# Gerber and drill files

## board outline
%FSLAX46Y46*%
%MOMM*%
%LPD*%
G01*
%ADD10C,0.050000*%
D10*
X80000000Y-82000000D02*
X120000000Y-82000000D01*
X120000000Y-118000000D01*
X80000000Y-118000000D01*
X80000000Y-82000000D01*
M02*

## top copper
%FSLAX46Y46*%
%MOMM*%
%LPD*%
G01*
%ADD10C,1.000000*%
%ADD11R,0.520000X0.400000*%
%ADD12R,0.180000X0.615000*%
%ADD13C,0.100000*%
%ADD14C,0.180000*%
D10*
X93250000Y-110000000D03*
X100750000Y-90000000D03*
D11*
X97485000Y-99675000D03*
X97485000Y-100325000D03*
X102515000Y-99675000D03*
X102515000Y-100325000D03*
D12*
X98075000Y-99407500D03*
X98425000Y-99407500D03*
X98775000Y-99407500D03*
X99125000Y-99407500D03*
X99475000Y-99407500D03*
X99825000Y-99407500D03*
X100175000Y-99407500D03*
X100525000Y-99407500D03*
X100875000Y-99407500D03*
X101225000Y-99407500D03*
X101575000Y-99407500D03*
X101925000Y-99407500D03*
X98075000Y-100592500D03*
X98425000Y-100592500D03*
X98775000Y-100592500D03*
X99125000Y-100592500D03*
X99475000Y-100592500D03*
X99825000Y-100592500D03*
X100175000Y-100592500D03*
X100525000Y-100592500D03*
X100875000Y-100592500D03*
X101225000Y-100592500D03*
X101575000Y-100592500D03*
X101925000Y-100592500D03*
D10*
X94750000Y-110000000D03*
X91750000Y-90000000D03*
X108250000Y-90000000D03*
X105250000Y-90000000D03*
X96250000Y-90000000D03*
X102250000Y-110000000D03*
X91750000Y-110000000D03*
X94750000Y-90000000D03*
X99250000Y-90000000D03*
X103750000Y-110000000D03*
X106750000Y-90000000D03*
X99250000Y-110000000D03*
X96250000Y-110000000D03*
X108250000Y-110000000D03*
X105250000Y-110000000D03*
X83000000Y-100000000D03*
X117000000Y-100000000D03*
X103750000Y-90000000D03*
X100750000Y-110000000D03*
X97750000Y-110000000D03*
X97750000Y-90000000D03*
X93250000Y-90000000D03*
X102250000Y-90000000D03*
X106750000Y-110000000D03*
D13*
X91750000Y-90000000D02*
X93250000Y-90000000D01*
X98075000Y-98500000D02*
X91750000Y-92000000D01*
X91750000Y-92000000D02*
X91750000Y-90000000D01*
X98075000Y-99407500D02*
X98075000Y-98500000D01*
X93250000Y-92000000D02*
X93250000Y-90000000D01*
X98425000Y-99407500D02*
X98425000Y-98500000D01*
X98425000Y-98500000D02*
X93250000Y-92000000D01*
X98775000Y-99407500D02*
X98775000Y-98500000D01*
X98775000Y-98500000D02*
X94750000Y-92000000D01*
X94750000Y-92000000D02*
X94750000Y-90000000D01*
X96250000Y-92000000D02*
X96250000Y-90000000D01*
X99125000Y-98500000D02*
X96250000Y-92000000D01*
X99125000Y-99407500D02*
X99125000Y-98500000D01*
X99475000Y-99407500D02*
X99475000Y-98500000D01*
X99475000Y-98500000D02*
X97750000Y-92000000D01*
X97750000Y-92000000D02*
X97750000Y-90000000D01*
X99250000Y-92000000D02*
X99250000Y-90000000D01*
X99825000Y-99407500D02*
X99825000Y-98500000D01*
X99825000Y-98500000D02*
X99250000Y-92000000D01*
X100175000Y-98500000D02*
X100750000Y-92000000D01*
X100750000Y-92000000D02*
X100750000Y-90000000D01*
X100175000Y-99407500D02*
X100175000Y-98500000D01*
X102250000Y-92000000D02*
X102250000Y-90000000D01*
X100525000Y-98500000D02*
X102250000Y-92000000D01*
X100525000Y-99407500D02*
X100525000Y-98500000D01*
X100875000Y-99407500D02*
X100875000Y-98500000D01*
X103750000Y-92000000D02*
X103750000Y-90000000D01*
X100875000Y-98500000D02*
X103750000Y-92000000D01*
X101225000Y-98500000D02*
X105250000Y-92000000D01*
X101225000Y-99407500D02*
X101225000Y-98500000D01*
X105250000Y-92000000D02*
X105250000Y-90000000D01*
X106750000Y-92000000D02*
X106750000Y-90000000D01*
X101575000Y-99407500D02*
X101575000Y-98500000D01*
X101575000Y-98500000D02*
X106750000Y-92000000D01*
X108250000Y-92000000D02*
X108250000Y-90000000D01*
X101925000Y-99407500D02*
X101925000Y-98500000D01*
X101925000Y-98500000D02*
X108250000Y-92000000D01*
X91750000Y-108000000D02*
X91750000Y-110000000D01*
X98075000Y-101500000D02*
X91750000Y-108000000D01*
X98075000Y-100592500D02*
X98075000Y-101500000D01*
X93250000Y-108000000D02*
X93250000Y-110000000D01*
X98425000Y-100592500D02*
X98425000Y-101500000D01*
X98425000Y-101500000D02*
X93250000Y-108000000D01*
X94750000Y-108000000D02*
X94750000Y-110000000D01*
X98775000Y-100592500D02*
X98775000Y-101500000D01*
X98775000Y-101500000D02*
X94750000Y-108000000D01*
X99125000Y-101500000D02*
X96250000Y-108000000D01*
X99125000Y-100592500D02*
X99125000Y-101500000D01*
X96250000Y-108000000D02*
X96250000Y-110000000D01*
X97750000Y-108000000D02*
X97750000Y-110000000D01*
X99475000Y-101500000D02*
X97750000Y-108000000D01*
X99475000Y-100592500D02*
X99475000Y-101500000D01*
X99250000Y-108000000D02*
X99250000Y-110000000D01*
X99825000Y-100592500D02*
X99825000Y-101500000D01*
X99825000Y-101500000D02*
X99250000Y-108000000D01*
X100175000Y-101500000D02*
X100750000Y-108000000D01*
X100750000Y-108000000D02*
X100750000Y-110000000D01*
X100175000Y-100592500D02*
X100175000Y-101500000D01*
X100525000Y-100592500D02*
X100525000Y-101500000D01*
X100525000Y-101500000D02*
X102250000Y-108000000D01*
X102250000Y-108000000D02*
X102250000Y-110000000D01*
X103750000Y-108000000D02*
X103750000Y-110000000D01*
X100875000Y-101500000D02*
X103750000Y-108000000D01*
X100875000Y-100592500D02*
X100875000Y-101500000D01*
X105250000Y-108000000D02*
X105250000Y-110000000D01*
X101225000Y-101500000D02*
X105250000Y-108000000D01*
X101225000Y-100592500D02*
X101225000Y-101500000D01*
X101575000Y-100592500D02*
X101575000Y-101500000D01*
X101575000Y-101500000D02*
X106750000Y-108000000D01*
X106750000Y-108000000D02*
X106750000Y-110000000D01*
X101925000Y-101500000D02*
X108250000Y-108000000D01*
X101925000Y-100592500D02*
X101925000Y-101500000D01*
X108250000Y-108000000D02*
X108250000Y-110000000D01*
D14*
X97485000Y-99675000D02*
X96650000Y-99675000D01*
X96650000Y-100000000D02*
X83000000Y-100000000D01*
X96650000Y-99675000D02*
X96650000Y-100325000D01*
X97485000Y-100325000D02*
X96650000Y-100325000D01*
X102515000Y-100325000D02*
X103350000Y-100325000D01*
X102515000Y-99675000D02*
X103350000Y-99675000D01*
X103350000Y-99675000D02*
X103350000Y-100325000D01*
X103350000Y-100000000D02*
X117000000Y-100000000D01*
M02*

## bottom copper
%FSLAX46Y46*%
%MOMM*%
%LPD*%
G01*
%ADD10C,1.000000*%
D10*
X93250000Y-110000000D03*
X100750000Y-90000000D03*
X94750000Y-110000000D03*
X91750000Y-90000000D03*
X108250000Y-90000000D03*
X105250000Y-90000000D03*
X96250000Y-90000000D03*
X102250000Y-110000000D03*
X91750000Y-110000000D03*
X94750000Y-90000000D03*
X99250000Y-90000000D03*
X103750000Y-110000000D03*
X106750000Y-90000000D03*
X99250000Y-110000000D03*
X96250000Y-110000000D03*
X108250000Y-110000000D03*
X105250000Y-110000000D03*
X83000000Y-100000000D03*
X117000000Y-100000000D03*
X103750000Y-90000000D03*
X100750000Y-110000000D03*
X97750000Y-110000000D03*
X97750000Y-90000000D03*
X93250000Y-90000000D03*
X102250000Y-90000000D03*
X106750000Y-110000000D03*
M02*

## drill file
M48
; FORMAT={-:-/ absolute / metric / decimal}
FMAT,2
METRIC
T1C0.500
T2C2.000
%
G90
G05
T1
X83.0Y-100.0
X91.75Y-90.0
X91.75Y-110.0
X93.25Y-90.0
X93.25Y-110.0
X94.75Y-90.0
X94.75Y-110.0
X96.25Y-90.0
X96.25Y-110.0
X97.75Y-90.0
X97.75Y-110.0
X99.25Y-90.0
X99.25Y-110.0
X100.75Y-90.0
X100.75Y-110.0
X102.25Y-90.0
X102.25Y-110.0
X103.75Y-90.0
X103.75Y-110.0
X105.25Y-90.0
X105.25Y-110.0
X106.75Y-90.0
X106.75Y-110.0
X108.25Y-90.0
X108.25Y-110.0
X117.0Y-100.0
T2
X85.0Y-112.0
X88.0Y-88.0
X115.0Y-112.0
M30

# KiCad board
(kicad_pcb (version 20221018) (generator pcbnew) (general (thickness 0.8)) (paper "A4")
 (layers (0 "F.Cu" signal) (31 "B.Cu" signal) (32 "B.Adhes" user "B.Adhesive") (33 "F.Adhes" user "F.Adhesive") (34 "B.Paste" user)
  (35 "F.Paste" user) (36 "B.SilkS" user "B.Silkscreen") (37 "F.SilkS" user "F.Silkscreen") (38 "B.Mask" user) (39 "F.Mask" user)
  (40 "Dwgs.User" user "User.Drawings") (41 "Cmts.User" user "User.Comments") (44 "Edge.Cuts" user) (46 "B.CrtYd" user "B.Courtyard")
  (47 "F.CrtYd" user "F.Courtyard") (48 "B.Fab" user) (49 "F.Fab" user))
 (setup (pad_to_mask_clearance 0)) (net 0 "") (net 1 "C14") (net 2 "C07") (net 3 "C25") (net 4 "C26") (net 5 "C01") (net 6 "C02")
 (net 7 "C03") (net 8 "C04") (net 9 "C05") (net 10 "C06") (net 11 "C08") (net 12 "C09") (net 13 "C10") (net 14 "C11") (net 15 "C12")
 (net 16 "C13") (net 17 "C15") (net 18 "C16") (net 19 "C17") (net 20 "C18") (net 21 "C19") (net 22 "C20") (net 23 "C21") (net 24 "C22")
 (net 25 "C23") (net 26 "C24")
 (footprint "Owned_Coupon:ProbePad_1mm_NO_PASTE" (layer "F.Cu") (at 93.25 110)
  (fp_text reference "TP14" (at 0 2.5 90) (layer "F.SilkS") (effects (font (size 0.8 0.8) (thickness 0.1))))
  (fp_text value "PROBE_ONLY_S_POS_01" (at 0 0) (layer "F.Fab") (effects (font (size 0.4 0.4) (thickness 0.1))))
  (pad "1" thru_hole circle (at 0 0) (size 1 1) (drill 0.5) (layers "*.Cu" "*.Mask") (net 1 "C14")))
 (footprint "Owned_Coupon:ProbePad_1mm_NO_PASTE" (layer "F.Cu") (at 100.75 90)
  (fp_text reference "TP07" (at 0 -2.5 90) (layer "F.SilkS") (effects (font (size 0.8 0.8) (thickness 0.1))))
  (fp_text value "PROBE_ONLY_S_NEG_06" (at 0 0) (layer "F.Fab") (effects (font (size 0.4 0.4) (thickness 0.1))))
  (pad "1" thru_hole circle (at 0 0) (size 1 1) (drill 0.5) (layers "*.Cu" "*.Mask") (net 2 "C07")))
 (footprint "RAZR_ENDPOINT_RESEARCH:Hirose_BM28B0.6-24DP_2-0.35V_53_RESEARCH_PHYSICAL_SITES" (layer "F.Cu") (at 100 100)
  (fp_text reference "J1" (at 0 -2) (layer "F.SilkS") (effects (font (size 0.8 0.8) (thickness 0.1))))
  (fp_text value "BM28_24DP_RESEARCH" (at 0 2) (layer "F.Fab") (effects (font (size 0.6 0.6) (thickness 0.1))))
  (pad "P_L" smd rect (at -2.515 -0.325) (size 0.52 0.4) (layers "F.Cu" "F.Mask") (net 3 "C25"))
  (pad "P_L" smd rect (at -2.515 0.325) (size 0.52 0.4) (layers "F.Cu" "F.Mask") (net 3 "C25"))
  (pad "P_R" smd rect (at 2.515 -0.325) (size 0.52 0.4) (layers "F.Cu" "F.Mask") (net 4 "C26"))
  (pad "P_R" smd rect (at 2.515 0.325) (size 0.52 0.4) (layers "F.Cu" "F.Mask") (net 4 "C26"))
  (pad "S_NEG_00" smd rect (at -1.925 -0.5925) (size 0.18 0.615) (layers "F.Cu" "F.Mask") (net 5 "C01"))
  (pad "S_NEG_01" smd rect (at -1.575 -0.5925) (size 0.18 0.615) (layers "F.Cu" "F.Mask") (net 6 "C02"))
  (pad "S_NEG_02" smd rect (at -1.225 -0.5925) (size 0.18 0.615) (layers "F.Cu" "F.Mask") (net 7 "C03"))
  (pad "S_NEG_03" smd rect (at -0.875 -0.5925) (size 0.18 0.615) (layers "F.Cu" "F.Mask") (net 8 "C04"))
  (pad "S_NEG_04" smd rect (at -0.525 -0.5925) (size 0.18 0.615) (layers "F.Cu" "F.Mask") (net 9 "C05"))
  (pad "S_NEG_05" smd rect (at -0.175 -0.5925) (size 0.18 0.615) (layers "F.Cu" "F.Mask") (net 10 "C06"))
  (pad "S_NEG_06" smd rect (at 0.175 -0.5925) (size 0.18 0.615) (layers "F.Cu" "F.Mask") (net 2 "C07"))
  (pad "S_NEG_07" smd rect (at 0.525 -0.5925) (size 0.18 0.615) (layers "F.Cu" "F.Mask") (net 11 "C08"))
  (pad "S_NEG_08" smd rect (at 0.875 -0.5925) (size 0.18 0.615) (layers "F.Cu" "F.Mask") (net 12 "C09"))
  (pad "S_NEG_09" smd rect (at 1.225 -0.5925) (size 0.18 0.615) (layers "F.Cu" "F.Mask") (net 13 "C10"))
  (pad "S_NEG_10" smd rect (at 1.575 -0.5925) (size 0.18 0.615) (layers "F.Cu" "F.Mask") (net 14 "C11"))
  (pad "S_NEG_11" smd rect (at 1.925 -0.5925) (size 0.18 0.615) (layers "F.Cu" "F.Mask") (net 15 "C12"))
  (pad "S_POS_00" smd rect (at -1.925 0.5925) (size 0.18 0.615) (layers "F.Cu" "F.Mask") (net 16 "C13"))
  (pad "S_POS_01" smd rect (at -1.575 0.5925) (size 0.18 0.615) (layers "F.Cu" "F.Mask") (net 1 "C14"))
  (pad "S_POS_02" smd rect (at -1.225 0.5925) (size 0.18 0.615) (layers "F.Cu" "F.Mask") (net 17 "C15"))
  (pad "S_POS_03" smd rect (at -0.875 0.5925) (size 0.18 0.615) (layers "F.Cu" "F.Mask") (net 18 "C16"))
  (pad "S_POS_04" smd rect (at -0.525 0.5925) (size 0.18 0.615) (layers "F.Cu" "F.Mask") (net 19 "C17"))
  (pad "S_POS_05" smd rect (at -0.175 0.5925) (size 0.18 0.615) (layers "F.Cu" "F.Mask") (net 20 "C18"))
  (pad "S_POS_06" smd rect (at 0.175 0.5925) (size 0.18 0.615) (layers "F.Cu" "F.Mask") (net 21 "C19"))
  (pad "S_POS_07" smd rect (at 0.525 0.5925) (size 0.18 0.615) (layers "F.Cu" "F.Mask") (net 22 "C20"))
  (pad "S_POS_08" smd rect (at 0.875 0.5925) (size 0.18 0.615) (layers "F.Cu" "F.Mask") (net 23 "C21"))
  (pad "S_POS_09" smd rect (at 1.225 0.5925) (size 0.18 0.615) (layers "F.Cu" "F.Mask") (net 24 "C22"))
  (pad "S_POS_10" smd rect (at 1.575 0.5925) (size 0.18 0.615) (layers "F.Cu" "F.Mask") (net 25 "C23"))
  (pad "S_POS_11" smd rect (at 1.925 0.5925) (size 0.18 0.615) (layers "F.Cu" "F.Mask") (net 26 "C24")))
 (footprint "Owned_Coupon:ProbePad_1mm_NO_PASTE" (layer "F.Cu") (at 94.75 110)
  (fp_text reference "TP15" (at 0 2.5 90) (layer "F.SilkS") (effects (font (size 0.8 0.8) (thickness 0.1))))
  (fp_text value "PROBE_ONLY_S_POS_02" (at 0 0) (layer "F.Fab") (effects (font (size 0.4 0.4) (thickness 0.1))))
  (pad "1" thru_hole circle (at 0 0) (size 1 1) (drill 0.5) (layers "*.Cu" "*.Mask") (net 17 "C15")))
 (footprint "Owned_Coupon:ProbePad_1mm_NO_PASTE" (layer "F.Cu") (at 91.75 90)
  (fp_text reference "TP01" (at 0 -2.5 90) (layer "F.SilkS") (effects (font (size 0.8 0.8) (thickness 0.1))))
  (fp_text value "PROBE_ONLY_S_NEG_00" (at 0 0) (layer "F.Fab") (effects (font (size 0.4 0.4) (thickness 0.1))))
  (pad "1" thru_hole circle (at 0 0) (size 1 1) (drill 0.5) (layers "*.Cu" "*.Mask") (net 5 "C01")))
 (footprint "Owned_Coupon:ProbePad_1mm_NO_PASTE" (layer "F.Cu") (at 108.25 90)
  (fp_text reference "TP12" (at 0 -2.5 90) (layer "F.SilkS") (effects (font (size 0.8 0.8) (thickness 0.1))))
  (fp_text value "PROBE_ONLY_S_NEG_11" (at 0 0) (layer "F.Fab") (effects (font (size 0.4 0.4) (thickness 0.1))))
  (pad "1" thru_hole circle (at 0 0) (size 1 1) (drill 0.5) (layers "*.Cu" "*.Mask") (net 15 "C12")))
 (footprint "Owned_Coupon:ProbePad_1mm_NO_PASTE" (layer "F.Cu") (at 105.25 90)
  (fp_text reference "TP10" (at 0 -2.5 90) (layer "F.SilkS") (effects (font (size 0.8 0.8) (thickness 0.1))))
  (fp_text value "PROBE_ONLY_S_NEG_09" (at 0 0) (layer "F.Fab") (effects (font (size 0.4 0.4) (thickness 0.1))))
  (pad "1" thru_hole circle (at 0 0) (size 1 1) (drill 0.5) (layers "*.Cu" "*.Mask") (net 13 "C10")))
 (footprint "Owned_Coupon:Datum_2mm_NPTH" (layer "F.Cu") (at 88 88)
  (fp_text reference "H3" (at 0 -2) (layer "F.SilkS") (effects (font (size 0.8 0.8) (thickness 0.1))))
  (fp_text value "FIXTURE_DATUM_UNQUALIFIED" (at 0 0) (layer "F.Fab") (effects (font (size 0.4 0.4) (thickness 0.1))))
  (pad "" np_thru_hole circle (at 0 0) (size 2 2) (drill 2) (layers "*.Cu" "*.Mask")))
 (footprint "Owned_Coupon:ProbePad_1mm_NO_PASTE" (layer "F.Cu") (at 96.25 90)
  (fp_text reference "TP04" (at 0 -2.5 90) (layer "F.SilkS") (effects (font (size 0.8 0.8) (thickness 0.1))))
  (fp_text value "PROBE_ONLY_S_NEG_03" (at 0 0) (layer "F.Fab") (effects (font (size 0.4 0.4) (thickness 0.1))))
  (pad "1" thru_hole circle (at 0 0) (size 1 1) (drill 0.5) (layers "*.Cu" "*.Mask") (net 8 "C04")))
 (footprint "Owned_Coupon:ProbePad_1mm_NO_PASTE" (layer "F.Cu") (at 102.25 110)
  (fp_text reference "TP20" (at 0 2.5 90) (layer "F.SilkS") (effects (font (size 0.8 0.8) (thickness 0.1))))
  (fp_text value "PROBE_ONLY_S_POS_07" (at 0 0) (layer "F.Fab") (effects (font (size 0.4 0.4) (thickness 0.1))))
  (pad "1" thru_hole circle (at 0 0) (size 1 1) (drill 0.5) (layers "*.Cu" "*.Mask") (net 22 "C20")))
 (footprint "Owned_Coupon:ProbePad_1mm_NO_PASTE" (layer "F.Cu") (at 91.75 110)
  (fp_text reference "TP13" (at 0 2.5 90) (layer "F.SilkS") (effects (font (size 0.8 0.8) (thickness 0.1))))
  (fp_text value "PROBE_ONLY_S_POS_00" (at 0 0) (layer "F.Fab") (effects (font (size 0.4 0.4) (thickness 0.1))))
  (pad "1" thru_hole circle (at 0 0) (size 1 1) (drill 0.5) (layers "*.Cu" "*.Mask") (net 16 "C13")))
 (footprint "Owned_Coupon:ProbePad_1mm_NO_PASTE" (layer "F.Cu") (at 94.75 90)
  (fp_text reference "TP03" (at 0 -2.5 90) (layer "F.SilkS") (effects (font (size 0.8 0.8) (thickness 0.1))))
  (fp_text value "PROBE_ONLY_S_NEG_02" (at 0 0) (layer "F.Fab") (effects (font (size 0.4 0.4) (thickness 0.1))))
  (pad "1" thru_hole circle (at 0 0) (size 1 1) (drill 0.5) (layers "*.Cu" "*.Mask") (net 7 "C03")))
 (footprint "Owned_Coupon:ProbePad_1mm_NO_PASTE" (layer "F.Cu") (at 99.25 90)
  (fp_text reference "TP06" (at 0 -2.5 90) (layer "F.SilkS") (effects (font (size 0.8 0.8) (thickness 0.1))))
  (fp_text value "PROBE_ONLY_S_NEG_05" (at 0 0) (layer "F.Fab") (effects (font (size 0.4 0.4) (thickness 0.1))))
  (pad "1" thru_hole circle (at 0 0) (size 1 1) (drill 0.5) (layers "*.Cu" "*.Mask") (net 10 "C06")))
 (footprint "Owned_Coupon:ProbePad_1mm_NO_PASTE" (layer "F.Cu") (at 103.75 110)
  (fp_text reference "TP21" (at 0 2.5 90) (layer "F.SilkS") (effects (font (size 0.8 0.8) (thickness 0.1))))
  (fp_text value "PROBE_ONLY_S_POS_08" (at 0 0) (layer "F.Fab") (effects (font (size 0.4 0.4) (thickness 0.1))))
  (pad "1" thru_hole circle (at 0 0) (size 1 1) (drill 0.5) (layers "*.Cu" "*.Mask") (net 23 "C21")))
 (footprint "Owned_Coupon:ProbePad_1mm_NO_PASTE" (layer "F.Cu") (at 106.75 90)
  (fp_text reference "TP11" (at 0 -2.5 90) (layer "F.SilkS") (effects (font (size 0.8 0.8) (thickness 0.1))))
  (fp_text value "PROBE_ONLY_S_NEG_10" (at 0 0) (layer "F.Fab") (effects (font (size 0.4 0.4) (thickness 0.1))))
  (pad "1" thru_hole circle (at 0 0) (size 1 1) (drill 0.5) (layers "*.Cu" "*.Mask") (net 14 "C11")))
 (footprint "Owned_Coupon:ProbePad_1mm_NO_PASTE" (layer "F.Cu") (at 99.25 110)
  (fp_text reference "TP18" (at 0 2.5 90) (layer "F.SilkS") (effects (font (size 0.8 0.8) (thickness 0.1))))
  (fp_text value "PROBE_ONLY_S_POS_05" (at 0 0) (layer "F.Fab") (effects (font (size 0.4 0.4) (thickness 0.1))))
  (pad "1" thru_hole circle (at 0 0) (size 1 1) (drill 0.5) (layers "*.Cu" "*.Mask") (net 20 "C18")))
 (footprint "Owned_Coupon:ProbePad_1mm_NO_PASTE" (layer "F.Cu") (at 96.25 110)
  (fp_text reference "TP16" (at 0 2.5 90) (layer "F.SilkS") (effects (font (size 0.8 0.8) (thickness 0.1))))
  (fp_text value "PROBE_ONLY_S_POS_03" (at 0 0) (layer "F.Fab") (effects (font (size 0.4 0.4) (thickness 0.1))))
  (pad "1" thru_hole circle (at 0 0) (size 1 1) (drill 0.5) (layers "*.Cu" "*.Mask") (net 18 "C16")))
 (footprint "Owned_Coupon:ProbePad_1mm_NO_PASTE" (layer "F.Cu") (at 108.25 110)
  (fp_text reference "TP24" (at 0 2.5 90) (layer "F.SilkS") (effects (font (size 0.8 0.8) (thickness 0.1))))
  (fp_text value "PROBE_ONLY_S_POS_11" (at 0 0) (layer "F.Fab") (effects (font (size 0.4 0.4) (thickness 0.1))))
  (pad "1" thru_hole circle (at 0 0) (size 1 1) (drill 0.5) (layers "*.Cu" "*.Mask") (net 26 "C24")))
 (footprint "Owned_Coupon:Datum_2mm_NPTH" (layer "F.Cu") (at 85 112)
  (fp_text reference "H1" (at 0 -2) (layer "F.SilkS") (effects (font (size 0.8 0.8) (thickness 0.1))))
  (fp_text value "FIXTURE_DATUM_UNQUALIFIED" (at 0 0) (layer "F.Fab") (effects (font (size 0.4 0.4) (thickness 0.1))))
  (pad "" np_thru_hole circle (at 0 0) (size 2 2) (drill 2) (layers "*.Cu" "*.Mask")))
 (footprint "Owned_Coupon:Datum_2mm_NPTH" (layer "F.Cu") (at 115 112)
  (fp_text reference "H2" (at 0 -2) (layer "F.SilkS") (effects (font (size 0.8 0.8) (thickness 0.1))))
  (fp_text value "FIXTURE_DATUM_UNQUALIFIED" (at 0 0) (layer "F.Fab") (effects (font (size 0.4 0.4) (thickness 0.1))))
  (pad "" np_thru_hole circle (at 0 0) (size 2 2) (drill 2) (layers "*.Cu" "*.Mask")))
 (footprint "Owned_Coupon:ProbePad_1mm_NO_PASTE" (layer "F.Cu") (at 105.25 110)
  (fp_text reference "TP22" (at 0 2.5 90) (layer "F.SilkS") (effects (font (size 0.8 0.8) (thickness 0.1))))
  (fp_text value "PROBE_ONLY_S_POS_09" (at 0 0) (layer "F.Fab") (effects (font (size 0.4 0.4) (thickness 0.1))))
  (pad "1" thru_hole circle (at 0 0) (size 1 1) (drill 0.5) (layers "*.Cu" "*.Mask") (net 24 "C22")))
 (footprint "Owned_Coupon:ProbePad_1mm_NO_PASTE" (layer "F.Cu") (at 83 100)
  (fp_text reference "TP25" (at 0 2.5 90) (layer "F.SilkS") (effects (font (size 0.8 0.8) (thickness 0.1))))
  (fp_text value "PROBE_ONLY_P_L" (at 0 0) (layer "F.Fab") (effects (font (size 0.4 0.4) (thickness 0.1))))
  (pad "1" thru_hole circle (at 0 0) (size 1 1) (drill 0.5) (layers "*.Cu" "*.Mask") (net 3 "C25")))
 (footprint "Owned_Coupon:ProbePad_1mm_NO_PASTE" (layer "F.Cu") (at 117 100)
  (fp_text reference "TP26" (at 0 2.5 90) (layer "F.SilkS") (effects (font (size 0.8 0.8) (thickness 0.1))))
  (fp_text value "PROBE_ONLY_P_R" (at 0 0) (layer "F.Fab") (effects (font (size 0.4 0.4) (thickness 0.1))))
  (pad "1" thru_hole circle (at 0 0) (size 1 1) (drill 0.5) (layers "*.Cu" "*.Mask") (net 4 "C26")))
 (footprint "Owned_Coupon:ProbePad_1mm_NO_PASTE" (layer "F.Cu") (at 103.75 90)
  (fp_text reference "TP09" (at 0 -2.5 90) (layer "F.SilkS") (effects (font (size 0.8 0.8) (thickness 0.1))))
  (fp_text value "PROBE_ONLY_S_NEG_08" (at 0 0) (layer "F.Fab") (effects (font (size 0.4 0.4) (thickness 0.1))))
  (pad "1" thru_hole circle (at 0 0) (size 1 1) (drill 0.5) (layers "*.Cu" "*.Mask") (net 12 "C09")))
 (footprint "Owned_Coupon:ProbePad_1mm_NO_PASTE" (layer "F.Cu") (at 100.75 110)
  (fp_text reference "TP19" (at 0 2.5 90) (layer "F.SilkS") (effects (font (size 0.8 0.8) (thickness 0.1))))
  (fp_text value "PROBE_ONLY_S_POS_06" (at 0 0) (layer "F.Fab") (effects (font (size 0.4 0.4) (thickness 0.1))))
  (pad "1" thru_hole circle (at 0 0) (size 1 1) (drill 0.5) (layers "*.Cu" "*.Mask") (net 21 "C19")))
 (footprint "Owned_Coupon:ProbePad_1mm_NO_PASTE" (layer "F.Cu") (at 97.75 110)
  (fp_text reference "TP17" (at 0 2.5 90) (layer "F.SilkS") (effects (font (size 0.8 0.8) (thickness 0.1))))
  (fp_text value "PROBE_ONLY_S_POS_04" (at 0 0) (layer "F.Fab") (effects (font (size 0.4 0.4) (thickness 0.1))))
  (pad "1" thru_hole circle (at 0 0) (size 1 1) (drill 0.5) (layers "*.Cu" "*.Mask") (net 19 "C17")))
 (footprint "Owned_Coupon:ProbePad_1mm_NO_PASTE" (layer "F.Cu") (at 97.75 90)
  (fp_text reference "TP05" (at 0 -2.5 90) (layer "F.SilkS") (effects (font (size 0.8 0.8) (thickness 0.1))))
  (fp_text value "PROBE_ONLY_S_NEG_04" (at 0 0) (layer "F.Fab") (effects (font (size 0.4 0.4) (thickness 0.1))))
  (pad "1" thru_hole circle (at 0 0) (size 1 1) (drill 0.5) (layers "*.Cu" "*.Mask") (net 9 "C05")))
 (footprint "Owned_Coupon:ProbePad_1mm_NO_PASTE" (layer "F.Cu") (at 93.25 90)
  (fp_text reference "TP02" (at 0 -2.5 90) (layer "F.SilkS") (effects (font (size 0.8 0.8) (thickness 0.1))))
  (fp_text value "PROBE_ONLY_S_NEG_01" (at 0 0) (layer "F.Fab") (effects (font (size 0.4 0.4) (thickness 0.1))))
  (pad "1" thru_hole circle (at 0 0) (size 1 1) (drill 0.5) (layers "*.Cu" "*.Mask") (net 6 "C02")))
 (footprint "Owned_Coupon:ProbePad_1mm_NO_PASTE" (layer "F.Cu") (at 102.25 90)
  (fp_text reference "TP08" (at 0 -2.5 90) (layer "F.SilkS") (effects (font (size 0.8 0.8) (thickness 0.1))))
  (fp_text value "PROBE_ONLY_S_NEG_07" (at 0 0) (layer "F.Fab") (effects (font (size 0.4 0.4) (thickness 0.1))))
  (pad "1" thru_hole circle (at 0 0) (size 1 1) (drill 0.5) (layers "*.Cu" "*.Mask") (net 11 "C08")))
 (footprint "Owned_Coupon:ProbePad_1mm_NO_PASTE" (layer "F.Cu") (at 106.75 110)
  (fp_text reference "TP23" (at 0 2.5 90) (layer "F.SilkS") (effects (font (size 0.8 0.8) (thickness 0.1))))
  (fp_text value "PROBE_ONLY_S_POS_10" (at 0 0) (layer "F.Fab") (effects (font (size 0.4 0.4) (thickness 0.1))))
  (pad "1" thru_hole circle (at 0 0) (size 1 1) (drill 0.5) (layers "*.Cu" "*.Mask") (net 25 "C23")))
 (gr_rect (start 80 82) (end 120 118) (stroke (width 0.05) (type default)) (fill none) (layer "Edge.Cuts"))
 (segment (start 91.75 90) (end 93.25 90) (width 0.1) (layer "F.Cu") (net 5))
 (segment (start 98.075 98.5) (end 91.75 92) (width 0.1) (layer "F.Cu") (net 5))
 (segment (start 91.75 92) (end 91.75 90) (width 0.1) (layer "F.Cu") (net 5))
 (segment (start 98.075 99.4075) (end 98.075 98.5) (width 0.1) (layer "F.Cu") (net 5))
 (segment (start 93.25 92) (end 93.25 90) (width 0.1) (layer "F.Cu") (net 6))
 (segment (start 98.425 99.4075) (end 98.425 98.5) (width 0.1) (layer "F.Cu") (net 6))
 (segment (start 98.425 98.5) (end 93.25 92) (width 0.1) (layer "F.Cu") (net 6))
 (segment (start 98.775 99.4075) (end 98.775 98.5) (width 0.1) (layer "F.Cu") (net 7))
 (segment (start 98.775 98.5) (end 94.75 92) (width 0.1) (layer "F.Cu") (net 7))
 (segment (start 94.75 92) (end 94.75 90) (width 0.1) (layer "F.Cu") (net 7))
 (segment (start 96.25 92) (end 96.25 90) (width 0.1) (layer "F.Cu") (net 8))
 (segment (start 99.125 98.5) (end 96.25 92) (width 0.1) (layer "F.Cu") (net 8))
 (segment (start 99.125 99.4075) (end 99.125 98.5) (width 0.1) (layer "F.Cu") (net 8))
 (segment (start 99.475 99.4075) (end 99.475 98.5) (width 0.1) (layer "F.Cu") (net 9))
 (segment (start 99.475 98.5) (end 97.75 92) (width 0.1) (layer "F.Cu") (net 9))
 (segment (start 97.75 92) (end 97.75 90) (width 0.1) (layer "F.Cu") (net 9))
 (segment (start 99.25 92) (end 99.25 90) (width 0.1) (layer "F.Cu") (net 10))
 (segment (start 99.825 99.4075) (end 99.825 98.5) (width 0.1) (layer "F.Cu") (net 10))
 (segment (start 99.825 98.5) (end 99.25 92) (width 0.1) (layer "F.Cu") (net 10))
 (segment (start 100.175 98.5) (end 100.75 92) (width 0.1) (layer "F.Cu") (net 2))
 (segment (start 100.75 92) (end 100.75 90) (width 0.1) (layer "F.Cu") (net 2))
 (segment (start 100.175 99.4075) (end 100.175 98.5) (width 0.1) (layer "F.Cu") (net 2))
 (segment (start 102.25 92) (end 102.25 90) (width 0.1) (layer "F.Cu") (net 11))
 (segment (start 100.525 98.5) (end 102.25 92) (width 0.1) (layer "F.Cu") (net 11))
 (segment (start 100.525 99.4075) (end 100.525 98.5) (width 0.1) (layer "F.Cu") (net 11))
 (segment (start 100.875 99.4075) (end 100.875 98.5) (width 0.1) (layer "F.Cu") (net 12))
 (segment (start 103.75 92) (end 103.75 90) (width 0.1) (layer "F.Cu") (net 12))
 (segment (start 100.875 98.5) (end 103.75 92) (width 0.1) (layer "F.Cu") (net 12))
 (segment (start 101.225 98.5) (end 105.25 92) (width 0.1) (layer "F.Cu") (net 13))
 (segment (start 101.225 99.4075) (end 101.225 98.5) (width 0.1) (layer "F.Cu") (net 13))
 (segment (start 105.25 92) (end 105.25 90) (width 0.1) (layer "F.Cu") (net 13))
 (segment (start 106.75 92) (end 106.75 90) (width 0.1) (layer "F.Cu") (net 14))
 (segment (start 101.575 99.4075) (end 101.575 98.5) (width 0.1) (layer "F.Cu") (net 14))
 (segment (start 101.575 98.5) (end 106.75 92) (width 0.1) (layer "F.Cu") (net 14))
 (segment (start 108.25 92) (end 108.25 90) (width 0.1) (layer "F.Cu") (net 15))
 (segment (start 101.925 99.4075) (end 101.925 98.5) (width 0.1) (layer "F.Cu") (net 15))
 (segment (start 101.925 98.5) (end 108.25 92) (width 0.1) (layer "F.Cu") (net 15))
 (segment (start 91.75 108) (end 91.75 110) (width 0.1) (layer "F.Cu") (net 16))
 (segment (start 98.075 101.5) (end 91.75 108) (width 0.1) (layer "F.Cu") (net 16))
 (segment (start 98.075 100.5925) (end 98.075 101.5) (width 0.1) (layer "F.Cu") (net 16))
 (segment (start 93.25 108) (end 93.25 110) (width 0.1) (layer "F.Cu") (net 1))
 (segment (start 98.425 100.5925) (end 98.425 101.5) (width 0.1) (layer "F.Cu") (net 1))
 (segment (start 98.425 101.5) (end 93.25 108) (width 0.1) (layer "F.Cu") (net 1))
 (segment (start 94.75 108) (end 94.75 110) (width 0.1) (layer "F.Cu") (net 17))
 (segment (start 98.775 100.5925) (end 98.775 101.5) (width 0.1) (layer "F.Cu") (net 17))
 (segment (start 98.775 101.5) (end 94.75 108) (width 0.1) (layer "F.Cu") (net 17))
 (segment (start 99.125 101.5) (end 96.25 108) (width 0.1) (layer "F.Cu") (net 18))
 (segment (start 99.125 100.5925) (end 99.125 101.5) (width 0.1) (layer "F.Cu") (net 18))
 (segment (start 96.25 108) (end 96.25 110) (width 0.1) (layer "F.Cu") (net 18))
 (segment (start 97.75 108) (end 97.75 110) (width 0.1) (layer "F.Cu") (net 19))
 (segment (start 99.475 101.5) (end 97.75 108) (width 0.1) (layer "F.Cu") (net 19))
 (segment (start 99.475 100.5925) (end 99.475 101.5) (width 0.1) (layer "F.Cu") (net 19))
 (segment (start 99.25 108) (end 99.25 110) (width 0.1) (layer "F.Cu") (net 20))
 (segment (start 99.825 100.5925) (end 99.825 101.5) (width 0.1) (layer "F.Cu") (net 20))
 (segment (start 99.825 101.5) (end 99.25 108) (width 0.1) (layer "F.Cu") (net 20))
 (segment (start 100.175 101.5) (end 100.75 108) (width 0.1) (layer "F.Cu") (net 21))
 (segment (start 100.75 108) (end 100.75 110) (width 0.1) (layer "F.Cu") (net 21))
 (segment (start 100.175 100.5925) (end 100.175 101.5) (width 0.1) (layer "F.Cu") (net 21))
 (segment (start 100.525 100.5925) (end 100.525 101.5) (width 0.1) (layer "F.Cu") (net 22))
 (segment (start 100.525 101.5) (end 102.25 108) (width 0.1) (layer "F.Cu") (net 22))
 (segment (start 102.25 108) (end 102.25 110) (width 0.1) (layer "F.Cu") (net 22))
 (segment (start 103.75 108) (end 103.75 110) (width 0.1) (layer "F.Cu") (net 23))
 (segment (start 100.875 101.5) (end 103.75 108) (width 0.1) (layer "F.Cu") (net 23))
 (segment (start 100.875 100.5925) (end 100.875 101.5) (width 0.1) (layer "F.Cu") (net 23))
 (segment (start 105.25 108) (end 105.25 110) (width 0.1) (layer "F.Cu") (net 24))
 (segment (start 101.225 101.5) (end 105.25 108) (width 0.1) (layer "F.Cu") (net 24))
 (segment (start 101.225 100.5925) (end 101.225 101.5) (width 0.1) (layer "F.Cu") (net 24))
 (segment (start 101.575 100.5925) (end 101.575 101.5) (width 0.1) (layer "F.Cu") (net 25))
 (segment (start 101.575 101.5) (end 106.75 108) (width 0.1) (layer "F.Cu") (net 25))
 (segment (start 106.75 108) (end 106.75 110) (width 0.1) (layer "F.Cu") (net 25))
 (segment (start 101.925 101.5) (end 108.25 108) (width 0.1) (layer "F.Cu") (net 26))
 (segment (start 101.925 100.5925) (end 101.925 101.5) (width 0.1) (layer "F.Cu") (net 26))
 (segment (start 108.25 108) (end 108.25 110) (width 0.1) (layer "F.Cu") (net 26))
 (segment (start 97.485 99.675) (end 96.65 99.675) (width 0.18) (layer "F.Cu") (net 3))
 (segment (start 96.65 100) (end 83 100) (width 0.18) (layer "F.Cu") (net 3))
 (segment (start 96.65 99.675) (end 96.65 100.325) (width 0.18) (layer "F.Cu") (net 3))
 (segment (start 97.485 100.325) (end 96.65 100.325) (width 0.18) (layer "F.Cu") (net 3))
 (segment (start 102.515 100.325) (end 103.35 100.325) (width 0.18) (layer "F.Cu") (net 4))
 (segment (start 102.515 99.675) (end 103.35 99.675) (width 0.18) (layer "F.Cu") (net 4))
 (segment (start 103.35 99.675) (end 103.35 100.325) (width 0.18) (layer "F.Cu") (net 4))
 (segment (start 103.35 100) (end 117 100) (width 0.18) (layer "F.Cu") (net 4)))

